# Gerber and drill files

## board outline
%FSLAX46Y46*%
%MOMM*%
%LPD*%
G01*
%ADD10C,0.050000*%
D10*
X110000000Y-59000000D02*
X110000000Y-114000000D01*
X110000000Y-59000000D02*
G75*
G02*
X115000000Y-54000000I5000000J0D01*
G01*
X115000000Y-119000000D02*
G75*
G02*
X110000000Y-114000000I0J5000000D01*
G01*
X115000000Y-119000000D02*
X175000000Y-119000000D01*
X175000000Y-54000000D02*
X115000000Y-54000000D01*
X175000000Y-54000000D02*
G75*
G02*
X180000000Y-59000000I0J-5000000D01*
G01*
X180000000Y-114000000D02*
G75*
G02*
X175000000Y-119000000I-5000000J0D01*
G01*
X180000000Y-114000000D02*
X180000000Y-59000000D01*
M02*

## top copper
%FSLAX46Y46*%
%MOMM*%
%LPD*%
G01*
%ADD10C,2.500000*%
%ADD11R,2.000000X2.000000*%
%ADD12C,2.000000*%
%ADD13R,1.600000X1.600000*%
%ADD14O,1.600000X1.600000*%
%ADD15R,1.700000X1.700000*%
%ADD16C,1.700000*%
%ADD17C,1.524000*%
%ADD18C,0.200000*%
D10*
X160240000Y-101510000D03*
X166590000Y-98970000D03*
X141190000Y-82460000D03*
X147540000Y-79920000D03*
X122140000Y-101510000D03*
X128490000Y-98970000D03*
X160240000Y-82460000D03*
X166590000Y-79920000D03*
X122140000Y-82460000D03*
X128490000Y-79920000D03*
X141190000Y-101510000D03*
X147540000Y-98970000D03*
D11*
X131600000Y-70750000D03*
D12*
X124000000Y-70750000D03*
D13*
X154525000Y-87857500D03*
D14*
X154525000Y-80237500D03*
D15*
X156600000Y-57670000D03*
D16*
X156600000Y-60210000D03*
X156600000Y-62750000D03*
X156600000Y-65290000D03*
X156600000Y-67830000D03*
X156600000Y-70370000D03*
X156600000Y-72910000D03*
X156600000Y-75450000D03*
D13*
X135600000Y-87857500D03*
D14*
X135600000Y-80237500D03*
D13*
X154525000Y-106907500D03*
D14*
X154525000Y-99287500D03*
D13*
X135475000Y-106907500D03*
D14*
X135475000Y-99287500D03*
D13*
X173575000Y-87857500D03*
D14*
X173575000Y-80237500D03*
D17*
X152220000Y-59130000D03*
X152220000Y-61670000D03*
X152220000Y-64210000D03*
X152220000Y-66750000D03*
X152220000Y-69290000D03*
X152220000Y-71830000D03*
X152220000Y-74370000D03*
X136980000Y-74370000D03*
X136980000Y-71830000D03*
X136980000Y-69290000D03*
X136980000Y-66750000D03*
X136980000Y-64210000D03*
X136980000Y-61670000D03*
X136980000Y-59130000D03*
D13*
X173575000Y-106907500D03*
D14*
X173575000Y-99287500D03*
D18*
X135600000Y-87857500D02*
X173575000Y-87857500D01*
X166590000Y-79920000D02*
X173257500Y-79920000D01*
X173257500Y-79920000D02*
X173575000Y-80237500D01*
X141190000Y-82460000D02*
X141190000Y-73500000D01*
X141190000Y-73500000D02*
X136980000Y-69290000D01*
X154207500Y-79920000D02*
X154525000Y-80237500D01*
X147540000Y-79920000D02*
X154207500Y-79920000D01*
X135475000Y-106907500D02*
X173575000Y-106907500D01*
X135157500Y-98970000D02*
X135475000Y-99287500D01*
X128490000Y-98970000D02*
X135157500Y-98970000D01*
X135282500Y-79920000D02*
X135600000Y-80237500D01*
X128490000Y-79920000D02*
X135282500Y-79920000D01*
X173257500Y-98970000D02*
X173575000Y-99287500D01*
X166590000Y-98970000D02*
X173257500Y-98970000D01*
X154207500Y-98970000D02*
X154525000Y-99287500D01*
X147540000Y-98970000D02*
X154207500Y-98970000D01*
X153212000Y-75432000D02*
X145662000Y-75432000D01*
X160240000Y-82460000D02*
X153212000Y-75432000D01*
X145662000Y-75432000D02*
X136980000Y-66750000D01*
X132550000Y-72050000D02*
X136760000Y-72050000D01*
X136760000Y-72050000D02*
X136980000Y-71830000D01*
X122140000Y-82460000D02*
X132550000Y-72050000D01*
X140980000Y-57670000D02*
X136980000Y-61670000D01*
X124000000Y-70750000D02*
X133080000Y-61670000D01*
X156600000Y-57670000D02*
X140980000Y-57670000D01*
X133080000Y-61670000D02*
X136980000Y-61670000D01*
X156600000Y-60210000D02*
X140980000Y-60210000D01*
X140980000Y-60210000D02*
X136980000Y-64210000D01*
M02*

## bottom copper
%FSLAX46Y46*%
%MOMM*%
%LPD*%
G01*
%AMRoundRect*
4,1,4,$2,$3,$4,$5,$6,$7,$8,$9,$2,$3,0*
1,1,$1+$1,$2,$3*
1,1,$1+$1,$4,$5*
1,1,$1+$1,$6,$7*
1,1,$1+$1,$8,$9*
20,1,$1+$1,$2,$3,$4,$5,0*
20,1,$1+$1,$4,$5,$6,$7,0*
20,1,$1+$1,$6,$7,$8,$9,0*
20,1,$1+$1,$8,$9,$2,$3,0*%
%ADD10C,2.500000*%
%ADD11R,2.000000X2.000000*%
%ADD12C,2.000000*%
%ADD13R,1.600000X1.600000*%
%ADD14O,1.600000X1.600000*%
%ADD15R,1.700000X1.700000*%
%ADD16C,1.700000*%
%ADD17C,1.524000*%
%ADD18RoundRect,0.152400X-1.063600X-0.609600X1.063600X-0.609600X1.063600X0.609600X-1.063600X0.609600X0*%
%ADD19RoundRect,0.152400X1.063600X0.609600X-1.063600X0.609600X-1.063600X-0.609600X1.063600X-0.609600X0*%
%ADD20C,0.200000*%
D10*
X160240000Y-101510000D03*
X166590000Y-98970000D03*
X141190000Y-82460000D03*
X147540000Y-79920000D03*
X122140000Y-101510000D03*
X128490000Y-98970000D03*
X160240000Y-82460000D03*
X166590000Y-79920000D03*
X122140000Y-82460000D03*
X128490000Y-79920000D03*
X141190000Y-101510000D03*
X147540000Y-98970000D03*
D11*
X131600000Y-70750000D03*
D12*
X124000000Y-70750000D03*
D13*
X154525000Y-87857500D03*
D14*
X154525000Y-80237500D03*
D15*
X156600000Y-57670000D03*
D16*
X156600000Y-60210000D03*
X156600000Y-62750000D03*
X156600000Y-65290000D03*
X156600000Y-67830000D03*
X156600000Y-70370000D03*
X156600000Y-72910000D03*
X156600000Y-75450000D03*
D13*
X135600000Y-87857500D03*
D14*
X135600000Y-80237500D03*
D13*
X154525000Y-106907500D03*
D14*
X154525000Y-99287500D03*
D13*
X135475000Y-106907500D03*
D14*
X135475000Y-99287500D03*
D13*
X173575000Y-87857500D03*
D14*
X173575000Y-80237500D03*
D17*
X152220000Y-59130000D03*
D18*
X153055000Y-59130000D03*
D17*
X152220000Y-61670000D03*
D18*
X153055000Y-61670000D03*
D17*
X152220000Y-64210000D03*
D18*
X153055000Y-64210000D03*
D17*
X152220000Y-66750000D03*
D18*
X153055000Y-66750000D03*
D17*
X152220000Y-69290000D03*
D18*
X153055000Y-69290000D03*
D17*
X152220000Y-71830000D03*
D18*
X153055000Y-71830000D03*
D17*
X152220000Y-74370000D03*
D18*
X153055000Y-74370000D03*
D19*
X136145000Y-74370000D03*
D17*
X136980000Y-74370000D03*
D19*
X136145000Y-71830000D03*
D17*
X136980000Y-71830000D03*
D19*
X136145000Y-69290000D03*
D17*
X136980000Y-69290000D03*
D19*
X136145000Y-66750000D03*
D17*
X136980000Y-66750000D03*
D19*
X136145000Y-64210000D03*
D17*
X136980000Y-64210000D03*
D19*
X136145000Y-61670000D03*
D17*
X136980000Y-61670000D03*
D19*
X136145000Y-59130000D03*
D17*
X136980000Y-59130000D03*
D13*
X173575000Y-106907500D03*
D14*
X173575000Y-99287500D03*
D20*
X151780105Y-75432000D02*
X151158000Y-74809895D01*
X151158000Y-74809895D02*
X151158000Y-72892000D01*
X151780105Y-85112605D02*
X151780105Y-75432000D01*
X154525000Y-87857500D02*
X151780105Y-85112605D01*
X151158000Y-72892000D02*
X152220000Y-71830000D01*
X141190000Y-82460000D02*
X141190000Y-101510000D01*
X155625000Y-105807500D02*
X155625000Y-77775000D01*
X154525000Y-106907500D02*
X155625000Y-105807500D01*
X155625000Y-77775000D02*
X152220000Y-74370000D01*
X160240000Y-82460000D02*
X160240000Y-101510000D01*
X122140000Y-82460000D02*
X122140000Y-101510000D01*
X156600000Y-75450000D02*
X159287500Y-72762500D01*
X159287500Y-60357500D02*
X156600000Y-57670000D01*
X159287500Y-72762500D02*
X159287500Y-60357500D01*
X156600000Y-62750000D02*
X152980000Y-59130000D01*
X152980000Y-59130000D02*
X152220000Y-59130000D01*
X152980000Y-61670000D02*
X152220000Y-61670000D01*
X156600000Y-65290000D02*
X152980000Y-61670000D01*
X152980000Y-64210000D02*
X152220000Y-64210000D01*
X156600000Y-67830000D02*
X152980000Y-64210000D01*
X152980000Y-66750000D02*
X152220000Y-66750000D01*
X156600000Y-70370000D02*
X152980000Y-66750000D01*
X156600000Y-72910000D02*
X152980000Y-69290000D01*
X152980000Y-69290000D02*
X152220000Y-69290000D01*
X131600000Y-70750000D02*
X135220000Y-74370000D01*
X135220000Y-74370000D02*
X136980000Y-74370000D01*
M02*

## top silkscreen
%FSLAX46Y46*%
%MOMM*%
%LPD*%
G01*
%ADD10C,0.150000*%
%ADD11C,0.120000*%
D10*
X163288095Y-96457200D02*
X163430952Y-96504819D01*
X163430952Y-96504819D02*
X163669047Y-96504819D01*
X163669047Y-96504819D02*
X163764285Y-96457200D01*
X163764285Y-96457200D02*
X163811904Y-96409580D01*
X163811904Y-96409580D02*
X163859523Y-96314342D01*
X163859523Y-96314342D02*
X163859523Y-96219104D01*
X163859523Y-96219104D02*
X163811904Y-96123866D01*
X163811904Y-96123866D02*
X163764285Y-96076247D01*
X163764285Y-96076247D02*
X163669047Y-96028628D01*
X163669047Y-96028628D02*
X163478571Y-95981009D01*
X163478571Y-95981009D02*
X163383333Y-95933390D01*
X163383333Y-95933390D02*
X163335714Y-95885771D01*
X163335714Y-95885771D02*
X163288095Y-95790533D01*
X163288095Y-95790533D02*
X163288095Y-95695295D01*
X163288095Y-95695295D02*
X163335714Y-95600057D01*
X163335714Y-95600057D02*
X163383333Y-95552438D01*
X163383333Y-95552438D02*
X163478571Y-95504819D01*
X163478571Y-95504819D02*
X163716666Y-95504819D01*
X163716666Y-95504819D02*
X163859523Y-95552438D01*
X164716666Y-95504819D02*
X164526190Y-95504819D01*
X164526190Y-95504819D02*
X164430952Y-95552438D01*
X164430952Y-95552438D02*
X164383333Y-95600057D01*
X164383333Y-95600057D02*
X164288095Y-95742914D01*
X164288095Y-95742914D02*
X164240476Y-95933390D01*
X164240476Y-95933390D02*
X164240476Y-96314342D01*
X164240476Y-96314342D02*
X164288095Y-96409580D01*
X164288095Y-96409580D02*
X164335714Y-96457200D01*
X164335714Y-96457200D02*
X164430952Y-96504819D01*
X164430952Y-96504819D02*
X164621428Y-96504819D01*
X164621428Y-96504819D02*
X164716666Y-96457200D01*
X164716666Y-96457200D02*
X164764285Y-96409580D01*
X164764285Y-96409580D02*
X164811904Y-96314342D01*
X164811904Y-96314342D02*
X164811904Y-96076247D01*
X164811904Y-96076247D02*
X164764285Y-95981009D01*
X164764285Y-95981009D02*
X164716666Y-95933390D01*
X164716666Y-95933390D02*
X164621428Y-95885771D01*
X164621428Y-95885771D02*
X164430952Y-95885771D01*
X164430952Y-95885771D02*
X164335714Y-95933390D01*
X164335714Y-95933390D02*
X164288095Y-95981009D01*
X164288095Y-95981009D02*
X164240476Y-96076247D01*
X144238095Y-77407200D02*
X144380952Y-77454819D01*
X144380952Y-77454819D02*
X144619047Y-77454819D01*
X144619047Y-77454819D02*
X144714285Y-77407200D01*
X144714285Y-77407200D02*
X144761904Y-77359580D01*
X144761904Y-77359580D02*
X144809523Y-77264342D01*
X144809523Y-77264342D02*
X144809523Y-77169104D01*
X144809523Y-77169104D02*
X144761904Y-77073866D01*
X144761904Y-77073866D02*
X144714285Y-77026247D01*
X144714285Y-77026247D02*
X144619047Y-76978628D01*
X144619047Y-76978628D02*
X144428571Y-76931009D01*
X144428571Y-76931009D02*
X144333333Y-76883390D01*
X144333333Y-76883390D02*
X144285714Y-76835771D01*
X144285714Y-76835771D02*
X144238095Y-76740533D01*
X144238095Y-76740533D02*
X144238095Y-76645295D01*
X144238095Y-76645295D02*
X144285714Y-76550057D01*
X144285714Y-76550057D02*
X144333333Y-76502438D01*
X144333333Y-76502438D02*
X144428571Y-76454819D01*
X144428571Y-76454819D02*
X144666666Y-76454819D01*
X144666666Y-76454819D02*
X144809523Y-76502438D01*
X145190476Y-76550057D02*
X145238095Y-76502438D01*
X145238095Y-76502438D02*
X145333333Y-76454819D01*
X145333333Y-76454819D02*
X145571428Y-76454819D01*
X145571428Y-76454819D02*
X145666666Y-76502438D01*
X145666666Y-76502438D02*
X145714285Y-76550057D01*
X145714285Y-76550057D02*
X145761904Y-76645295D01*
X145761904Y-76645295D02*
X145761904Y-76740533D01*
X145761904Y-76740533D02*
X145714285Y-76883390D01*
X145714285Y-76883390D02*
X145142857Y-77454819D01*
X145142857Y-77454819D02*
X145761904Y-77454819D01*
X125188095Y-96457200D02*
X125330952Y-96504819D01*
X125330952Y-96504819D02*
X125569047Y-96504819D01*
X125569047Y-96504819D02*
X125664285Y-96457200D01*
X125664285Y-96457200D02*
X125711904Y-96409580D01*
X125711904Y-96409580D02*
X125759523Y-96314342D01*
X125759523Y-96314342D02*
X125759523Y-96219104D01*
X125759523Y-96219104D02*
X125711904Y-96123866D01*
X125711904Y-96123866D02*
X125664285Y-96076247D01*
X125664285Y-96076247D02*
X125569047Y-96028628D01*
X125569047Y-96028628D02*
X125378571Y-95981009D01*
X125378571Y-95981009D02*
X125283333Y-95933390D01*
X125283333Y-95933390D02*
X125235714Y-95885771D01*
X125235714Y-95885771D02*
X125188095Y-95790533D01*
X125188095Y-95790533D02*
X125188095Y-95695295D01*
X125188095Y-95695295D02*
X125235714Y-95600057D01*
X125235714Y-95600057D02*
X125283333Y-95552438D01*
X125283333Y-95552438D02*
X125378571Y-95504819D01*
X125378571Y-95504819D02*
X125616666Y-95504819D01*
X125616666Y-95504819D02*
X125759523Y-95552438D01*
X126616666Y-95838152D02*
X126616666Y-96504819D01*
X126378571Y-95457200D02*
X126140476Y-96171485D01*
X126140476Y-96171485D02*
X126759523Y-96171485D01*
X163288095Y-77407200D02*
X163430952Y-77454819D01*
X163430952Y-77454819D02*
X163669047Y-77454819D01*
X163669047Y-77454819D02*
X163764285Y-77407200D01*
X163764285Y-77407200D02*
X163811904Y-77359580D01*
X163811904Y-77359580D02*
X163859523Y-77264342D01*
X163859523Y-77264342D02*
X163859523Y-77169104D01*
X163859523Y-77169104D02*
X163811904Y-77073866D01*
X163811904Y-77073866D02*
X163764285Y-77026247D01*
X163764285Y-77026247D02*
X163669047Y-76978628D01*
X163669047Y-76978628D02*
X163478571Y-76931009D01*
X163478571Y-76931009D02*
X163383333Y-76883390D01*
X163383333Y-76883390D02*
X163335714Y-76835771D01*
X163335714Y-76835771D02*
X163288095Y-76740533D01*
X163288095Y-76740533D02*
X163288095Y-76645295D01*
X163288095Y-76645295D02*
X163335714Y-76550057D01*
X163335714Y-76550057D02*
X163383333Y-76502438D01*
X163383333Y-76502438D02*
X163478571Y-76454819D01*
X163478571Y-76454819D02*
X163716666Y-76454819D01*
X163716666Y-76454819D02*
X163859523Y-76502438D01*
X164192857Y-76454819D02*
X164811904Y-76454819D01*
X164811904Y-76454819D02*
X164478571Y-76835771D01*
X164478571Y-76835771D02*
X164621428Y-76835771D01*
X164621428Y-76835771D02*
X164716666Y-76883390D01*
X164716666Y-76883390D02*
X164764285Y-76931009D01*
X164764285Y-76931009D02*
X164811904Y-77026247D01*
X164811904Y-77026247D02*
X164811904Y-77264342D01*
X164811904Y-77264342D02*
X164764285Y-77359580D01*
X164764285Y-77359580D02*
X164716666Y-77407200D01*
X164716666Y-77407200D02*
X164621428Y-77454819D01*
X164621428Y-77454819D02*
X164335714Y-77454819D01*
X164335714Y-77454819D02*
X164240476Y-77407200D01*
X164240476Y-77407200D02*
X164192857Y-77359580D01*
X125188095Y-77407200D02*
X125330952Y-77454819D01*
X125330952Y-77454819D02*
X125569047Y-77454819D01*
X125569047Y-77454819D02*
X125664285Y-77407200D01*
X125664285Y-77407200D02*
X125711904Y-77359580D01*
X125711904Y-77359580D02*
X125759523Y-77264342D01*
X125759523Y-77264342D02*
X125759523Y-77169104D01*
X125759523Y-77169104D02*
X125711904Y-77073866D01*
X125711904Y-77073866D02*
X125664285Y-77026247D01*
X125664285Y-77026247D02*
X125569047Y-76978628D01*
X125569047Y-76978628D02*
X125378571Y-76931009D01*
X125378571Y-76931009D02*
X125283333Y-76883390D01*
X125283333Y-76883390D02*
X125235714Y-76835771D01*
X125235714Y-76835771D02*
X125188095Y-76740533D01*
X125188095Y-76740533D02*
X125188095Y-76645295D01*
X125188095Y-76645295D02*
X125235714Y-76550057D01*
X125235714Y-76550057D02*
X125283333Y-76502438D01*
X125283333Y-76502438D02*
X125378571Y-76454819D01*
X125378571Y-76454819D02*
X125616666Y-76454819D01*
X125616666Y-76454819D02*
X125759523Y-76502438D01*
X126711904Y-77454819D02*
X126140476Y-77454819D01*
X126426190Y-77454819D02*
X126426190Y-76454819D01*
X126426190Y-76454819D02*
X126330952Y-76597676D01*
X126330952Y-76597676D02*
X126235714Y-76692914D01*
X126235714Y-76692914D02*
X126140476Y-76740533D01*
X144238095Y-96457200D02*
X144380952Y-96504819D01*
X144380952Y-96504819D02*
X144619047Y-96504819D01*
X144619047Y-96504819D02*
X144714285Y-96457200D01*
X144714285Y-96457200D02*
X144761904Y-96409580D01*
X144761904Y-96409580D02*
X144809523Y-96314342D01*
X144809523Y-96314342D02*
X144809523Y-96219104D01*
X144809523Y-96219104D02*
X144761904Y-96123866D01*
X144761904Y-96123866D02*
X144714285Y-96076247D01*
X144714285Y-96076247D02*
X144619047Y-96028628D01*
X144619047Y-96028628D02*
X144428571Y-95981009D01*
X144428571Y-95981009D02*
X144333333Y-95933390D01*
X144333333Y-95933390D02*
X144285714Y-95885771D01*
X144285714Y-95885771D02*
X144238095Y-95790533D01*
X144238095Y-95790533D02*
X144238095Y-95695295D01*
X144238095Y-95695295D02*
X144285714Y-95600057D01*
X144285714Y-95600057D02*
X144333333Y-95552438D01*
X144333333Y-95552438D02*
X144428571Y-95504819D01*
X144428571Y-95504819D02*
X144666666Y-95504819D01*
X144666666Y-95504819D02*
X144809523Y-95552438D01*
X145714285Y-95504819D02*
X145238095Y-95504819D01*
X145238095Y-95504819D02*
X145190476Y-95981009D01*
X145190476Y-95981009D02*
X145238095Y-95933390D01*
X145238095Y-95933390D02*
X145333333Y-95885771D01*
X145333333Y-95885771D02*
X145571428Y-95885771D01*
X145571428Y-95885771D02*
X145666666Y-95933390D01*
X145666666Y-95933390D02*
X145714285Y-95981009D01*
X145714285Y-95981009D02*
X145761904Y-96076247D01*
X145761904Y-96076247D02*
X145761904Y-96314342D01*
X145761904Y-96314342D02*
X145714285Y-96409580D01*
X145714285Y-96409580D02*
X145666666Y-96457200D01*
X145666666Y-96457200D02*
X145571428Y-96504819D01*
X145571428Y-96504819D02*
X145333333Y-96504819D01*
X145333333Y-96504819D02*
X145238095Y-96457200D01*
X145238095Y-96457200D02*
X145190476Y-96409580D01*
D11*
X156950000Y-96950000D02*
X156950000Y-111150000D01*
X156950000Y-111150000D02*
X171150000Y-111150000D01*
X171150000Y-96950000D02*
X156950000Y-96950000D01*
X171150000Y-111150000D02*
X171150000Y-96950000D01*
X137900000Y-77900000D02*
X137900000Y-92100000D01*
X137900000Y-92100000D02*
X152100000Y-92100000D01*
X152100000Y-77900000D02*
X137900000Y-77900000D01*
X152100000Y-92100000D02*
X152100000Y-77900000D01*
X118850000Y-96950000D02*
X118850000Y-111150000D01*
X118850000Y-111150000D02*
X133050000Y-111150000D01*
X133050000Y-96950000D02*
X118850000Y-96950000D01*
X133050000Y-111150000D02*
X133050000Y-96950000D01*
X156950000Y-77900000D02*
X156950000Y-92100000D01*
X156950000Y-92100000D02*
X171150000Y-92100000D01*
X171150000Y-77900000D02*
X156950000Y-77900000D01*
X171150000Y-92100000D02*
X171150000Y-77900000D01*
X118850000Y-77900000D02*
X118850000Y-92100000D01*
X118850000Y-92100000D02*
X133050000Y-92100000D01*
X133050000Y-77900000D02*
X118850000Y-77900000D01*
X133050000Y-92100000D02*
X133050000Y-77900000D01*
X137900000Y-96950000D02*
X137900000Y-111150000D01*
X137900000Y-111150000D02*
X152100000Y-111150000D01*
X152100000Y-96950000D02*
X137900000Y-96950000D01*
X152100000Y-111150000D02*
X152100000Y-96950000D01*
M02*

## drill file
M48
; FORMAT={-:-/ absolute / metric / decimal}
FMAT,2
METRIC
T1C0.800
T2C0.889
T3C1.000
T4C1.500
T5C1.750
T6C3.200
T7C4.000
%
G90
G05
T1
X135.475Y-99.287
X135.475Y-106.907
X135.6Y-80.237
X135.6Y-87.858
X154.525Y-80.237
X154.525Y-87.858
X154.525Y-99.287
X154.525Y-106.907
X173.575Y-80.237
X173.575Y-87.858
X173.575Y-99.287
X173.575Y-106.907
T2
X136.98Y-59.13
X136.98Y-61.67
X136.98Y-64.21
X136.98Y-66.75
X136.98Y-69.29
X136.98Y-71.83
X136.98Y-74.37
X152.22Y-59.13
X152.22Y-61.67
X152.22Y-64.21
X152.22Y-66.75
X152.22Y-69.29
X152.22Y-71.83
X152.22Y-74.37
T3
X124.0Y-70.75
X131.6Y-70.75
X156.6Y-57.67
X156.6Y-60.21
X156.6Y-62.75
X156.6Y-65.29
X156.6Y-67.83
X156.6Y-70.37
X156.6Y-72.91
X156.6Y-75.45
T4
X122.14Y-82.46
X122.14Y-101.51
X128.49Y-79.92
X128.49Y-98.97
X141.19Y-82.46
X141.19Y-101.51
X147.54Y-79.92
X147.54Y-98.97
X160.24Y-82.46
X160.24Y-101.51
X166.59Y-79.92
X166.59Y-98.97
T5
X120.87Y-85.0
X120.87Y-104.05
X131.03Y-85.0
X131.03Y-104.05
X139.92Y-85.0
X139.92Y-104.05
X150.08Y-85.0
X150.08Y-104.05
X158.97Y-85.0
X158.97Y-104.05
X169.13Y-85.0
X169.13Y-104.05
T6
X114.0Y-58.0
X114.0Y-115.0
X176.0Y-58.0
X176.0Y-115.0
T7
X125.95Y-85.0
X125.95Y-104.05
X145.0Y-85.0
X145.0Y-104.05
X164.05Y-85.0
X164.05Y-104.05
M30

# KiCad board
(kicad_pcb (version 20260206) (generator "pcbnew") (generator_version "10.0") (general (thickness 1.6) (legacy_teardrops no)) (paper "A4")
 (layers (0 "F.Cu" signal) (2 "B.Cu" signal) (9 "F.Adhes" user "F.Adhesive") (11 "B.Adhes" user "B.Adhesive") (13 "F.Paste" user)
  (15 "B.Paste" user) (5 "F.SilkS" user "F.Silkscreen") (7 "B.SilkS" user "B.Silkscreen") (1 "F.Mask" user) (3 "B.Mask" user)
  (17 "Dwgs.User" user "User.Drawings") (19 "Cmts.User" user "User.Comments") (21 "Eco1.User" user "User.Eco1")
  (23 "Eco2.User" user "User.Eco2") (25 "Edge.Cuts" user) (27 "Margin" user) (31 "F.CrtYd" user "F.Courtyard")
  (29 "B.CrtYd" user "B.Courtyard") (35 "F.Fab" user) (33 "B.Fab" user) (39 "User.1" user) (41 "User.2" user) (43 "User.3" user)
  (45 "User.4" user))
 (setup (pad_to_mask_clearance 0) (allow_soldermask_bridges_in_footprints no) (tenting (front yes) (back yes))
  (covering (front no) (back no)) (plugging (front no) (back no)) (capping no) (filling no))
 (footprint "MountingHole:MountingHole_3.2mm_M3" (layer "F.Cu") (at 176 58)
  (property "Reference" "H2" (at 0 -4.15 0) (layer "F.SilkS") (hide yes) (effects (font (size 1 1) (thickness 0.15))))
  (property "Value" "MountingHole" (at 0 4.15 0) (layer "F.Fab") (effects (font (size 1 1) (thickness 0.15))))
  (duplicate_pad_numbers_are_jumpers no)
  (pad "" np_thru_hole circle (at 0 0) (size 3.2 3.2) (drill 3.2) (layers "*.Cu" "*.Mask")))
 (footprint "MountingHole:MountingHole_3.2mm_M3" (layer "F.Cu") (at 114 58)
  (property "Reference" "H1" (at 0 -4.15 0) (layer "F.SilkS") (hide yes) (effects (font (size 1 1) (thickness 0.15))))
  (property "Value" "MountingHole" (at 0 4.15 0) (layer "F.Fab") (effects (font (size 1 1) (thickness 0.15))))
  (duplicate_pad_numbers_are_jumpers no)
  (pad "" np_thru_hole circle (at 0 0) (size 3.2 3.2) (drill 3.2) (layers "*.Cu" "*.Mask")))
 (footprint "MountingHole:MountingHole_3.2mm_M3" (layer "F.Cu") (at 176 115)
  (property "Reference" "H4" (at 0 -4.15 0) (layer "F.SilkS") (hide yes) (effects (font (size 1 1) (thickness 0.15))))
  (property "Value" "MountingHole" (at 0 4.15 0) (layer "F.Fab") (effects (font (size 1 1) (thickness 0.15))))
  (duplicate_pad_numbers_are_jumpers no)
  (pad "" np_thru_hole circle (at 0 0) (size 3.2 3.2) (drill 3.2) (layers "*.Cu" "*.Mask")))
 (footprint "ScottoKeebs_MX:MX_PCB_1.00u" (layer "F.Cu") (at 164.05 104.05)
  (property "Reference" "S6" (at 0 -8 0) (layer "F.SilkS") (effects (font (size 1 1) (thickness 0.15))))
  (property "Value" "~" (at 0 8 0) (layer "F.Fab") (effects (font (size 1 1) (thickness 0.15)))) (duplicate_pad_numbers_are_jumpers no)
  (fp_line (start -7.1 -7.1) (end -7.1 7.1) (stroke (width 0.12) (type solid)) (layer "F.SilkS"))
  (fp_line (start -7.1 7.1) (end 7.1 7.1) (stroke (width 0.12) (type solid)) (layer "F.SilkS"))
  (fp_line (start 7.1 -7.1) (end -7.1 -7.1) (stroke (width 0.12) (type solid)) (layer "F.SilkS"))
  (fp_line (start 7.1 7.1) (end 7.1 -7.1) (stroke (width 0.12) (type solid)) (layer "F.SilkS"))
  (pad "" np_thru_hole circle (at -5.08 0) (size 1.75 1.75) (drill 1.75) (layers "*.Cu" "*.Mask"))
  (pad "" np_thru_hole circle (at 0 0) (size 4 4) (drill 4) (layers "*.Cu" "*.Mask"))
  (pad "" np_thru_hole circle (at 5.08 0) (size 1.75 1.75) (drill 1.75) (layers "*.Cu" "*.Mask"))
  (pad "1" thru_hole circle (at -3.81 -2.54) (size 2.5 2.5) (drill 1.5) (layers "*.Cu" "*.Mask") (remove_unused_layers no) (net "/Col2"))
  (pad "2" thru_hole circle (at 2.54 -5.08) (size 2.5 2.5) (drill 1.5) (layers "*.Cu" "*.Mask") (remove_unused_layers no) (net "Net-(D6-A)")))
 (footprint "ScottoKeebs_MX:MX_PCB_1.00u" (layer "F.Cu") (at 145 85)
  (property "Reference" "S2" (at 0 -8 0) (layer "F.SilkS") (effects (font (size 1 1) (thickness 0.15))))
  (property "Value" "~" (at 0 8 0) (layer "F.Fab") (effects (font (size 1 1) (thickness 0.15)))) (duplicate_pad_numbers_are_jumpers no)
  (fp_line (start -7.1 -7.1) (end -7.1 7.1) (stroke (width 0.12) (type solid)) (layer "F.SilkS"))
  (fp_line (start -7.1 7.1) (end 7.1 7.1) (stroke (width 0.12) (type solid)) (layer "F.SilkS"))
  (fp_line (start 7.1 -7.1) (end -7.1 -7.1) (stroke (width 0.12) (type solid)) (layer "F.SilkS"))
  (fp_line (start 7.1 7.1) (end 7.1 -7.1) (stroke (width 0.12) (type solid)) (layer "F.SilkS"))
  (pad "" np_thru_hole circle (at -5.08 0) (size 1.75 1.75) (drill 1.75) (layers "*.Cu" "*.Mask"))
  (pad "" np_thru_hole circle (at 0 0) (size 4 4) (drill 4) (layers "*.Cu" "*.Mask"))
  (pad "" np_thru_hole circle (at 5.08 0) (size 1.75 1.75) (drill 1.75) (layers "*.Cu" "*.Mask"))
  (pad "1" thru_hole circle (at -3.81 -2.54) (size 2.5 2.5) (drill 1.5) (layers "*.Cu" "*.Mask") (remove_unused_layers no) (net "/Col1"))
  (pad "2" thru_hole circle (at 2.54 -5.08) (size 2.5 2.5) (drill 1.5) (layers "*.Cu" "*.Mask") (remove_unused_layers no) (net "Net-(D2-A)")))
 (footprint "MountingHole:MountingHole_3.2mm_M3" (layer "F.Cu") (at 114 115)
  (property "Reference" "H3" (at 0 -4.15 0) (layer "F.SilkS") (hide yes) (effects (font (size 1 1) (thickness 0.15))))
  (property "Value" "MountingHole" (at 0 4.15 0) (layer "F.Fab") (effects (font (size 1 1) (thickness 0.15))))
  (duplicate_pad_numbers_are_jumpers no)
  (pad "" np_thru_hole circle (at 0 0) (size 3.2 3.2) (drill 3.2) (layers "*.Cu" "*.Mask")))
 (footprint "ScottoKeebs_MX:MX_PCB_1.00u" (layer "F.Cu") (at 125.95 104.05)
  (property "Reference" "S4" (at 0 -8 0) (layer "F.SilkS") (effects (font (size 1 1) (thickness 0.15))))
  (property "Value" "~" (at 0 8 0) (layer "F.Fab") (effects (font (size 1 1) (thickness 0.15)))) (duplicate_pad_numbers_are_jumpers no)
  (fp_line (start -7.1 -7.1) (end -7.1 7.1) (stroke (width 0.12) (type solid)) (layer "F.SilkS"))
  (fp_line (start -7.1 7.1) (end 7.1 7.1) (stroke (width 0.12) (type solid)) (layer "F.SilkS"))
  (fp_line (start 7.1 -7.1) (end -7.1 -7.1) (stroke (width 0.12) (type solid)) (layer "F.SilkS"))
  (fp_line (start 7.1 7.1) (end 7.1 -7.1) (stroke (width 0.12) (type solid)) (layer "F.SilkS"))
  (pad "" np_thru_hole circle (at -5.08 0) (size 1.75 1.75) (drill 1.75) (layers "*.Cu" "*.Mask"))
  (pad "" np_thru_hole circle (at 0 0) (size 4 4) (drill 4) (layers "*.Cu" "*.Mask"))
  (pad "" np_thru_hole circle (at 5.08 0) (size 1.75 1.75) (drill 1.75) (layers "*.Cu" "*.Mask"))
  (pad "1" thru_hole circle (at -3.81 -2.54) (size 2.5 2.5) (drill 1.5) (layers "*.Cu" "*.Mask") (remove_unused_layers no) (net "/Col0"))
  (pad "2" thru_hole circle (at 2.54 -5.08) (size 2.5 2.5) (drill 1.5) (layers "*.Cu" "*.Mask") (remove_unused_layers no) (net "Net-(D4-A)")))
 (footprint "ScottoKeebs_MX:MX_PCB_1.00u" (layer "F.Cu") (at 164.05 85)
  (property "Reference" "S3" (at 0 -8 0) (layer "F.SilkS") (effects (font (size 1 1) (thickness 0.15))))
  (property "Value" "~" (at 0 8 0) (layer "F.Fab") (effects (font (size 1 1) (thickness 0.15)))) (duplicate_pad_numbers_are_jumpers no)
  (fp_line (start -7.1 -7.1) (end -7.1 7.1) (stroke (width 0.12) (type solid)) (layer "F.SilkS"))
  (fp_line (start -7.1 7.1) (end 7.1 7.1) (stroke (width 0.12) (type solid)) (layer "F.SilkS"))
  (fp_line (start 7.1 -7.1) (end -7.1 -7.1) (stroke (width 0.12) (type solid)) (layer "F.SilkS"))
  (fp_line (start 7.1 7.1) (end 7.1 -7.1) (stroke (width 0.12) (type solid)) (layer "F.SilkS"))
  (pad "" np_thru_hole circle (at -5.08 0) (size 1.75 1.75) (drill 1.75) (layers "*.Cu" "*.Mask"))
  (pad "" np_thru_hole circle (at 0 0) (size 4 4) (drill 4) (layers "*.Cu" "*.Mask"))
  (pad "" np_thru_hole circle (at 5.08 0) (size 1.75 1.75) (drill 1.75) (layers "*.Cu" "*.Mask"))
  (pad "1" thru_hole circle (at -3.81 -2.54) (size 2.5 2.5) (drill 1.5) (layers "*.Cu" "*.Mask") (remove_unused_layers no) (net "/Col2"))
  (pad "2" thru_hole circle (at 2.54 -5.08) (size 2.5 2.5) (drill 1.5) (layers "*.Cu" "*.Mask") (remove_unused_layers no) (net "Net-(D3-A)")))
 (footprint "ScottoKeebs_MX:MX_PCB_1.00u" (layer "F.Cu") (at 125.95 85)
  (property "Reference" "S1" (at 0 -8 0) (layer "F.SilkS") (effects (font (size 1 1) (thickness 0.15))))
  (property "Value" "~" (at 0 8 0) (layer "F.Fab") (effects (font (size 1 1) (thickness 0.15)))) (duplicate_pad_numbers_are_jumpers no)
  (fp_line (start -7.1 -7.1) (end -7.1 7.1) (stroke (width 0.12) (type solid)) (layer "F.SilkS"))
  (fp_line (start -7.1 7.1) (end 7.1 7.1) (stroke (width 0.12) (type solid)) (layer "F.SilkS"))
  (fp_line (start 7.1 -7.1) (end -7.1 -7.1) (stroke (width 0.12) (type solid)) (layer "F.SilkS"))
  (fp_line (start 7.1 7.1) (end 7.1 -7.1) (stroke (width 0.12) (type solid)) (layer "F.SilkS"))
  (pad "" np_thru_hole circle (at -5.08 0) (size 1.75 1.75) (drill 1.75) (layers "*.Cu" "*.Mask"))
  (pad "" np_thru_hole circle (at 0 0) (size 4 4) (drill 4) (layers "*.Cu" "*.Mask"))
  (pad "" np_thru_hole circle (at 5.08 0) (size 1.75 1.75) (drill 1.75) (layers "*.Cu" "*.Mask"))
  (pad "1" thru_hole circle (at -3.81 -2.54) (size 2.5 2.5) (drill 1.5) (layers "*.Cu" "*.Mask") (remove_unused_layers no) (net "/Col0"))
  (pad "2" thru_hole circle (at 2.54 -5.08) (size 2.5 2.5) (drill 1.5) (layers "*.Cu" "*.Mask") (remove_unused_layers no) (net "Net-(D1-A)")))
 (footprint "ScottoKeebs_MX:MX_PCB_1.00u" (layer "F.Cu") (at 145 104.05)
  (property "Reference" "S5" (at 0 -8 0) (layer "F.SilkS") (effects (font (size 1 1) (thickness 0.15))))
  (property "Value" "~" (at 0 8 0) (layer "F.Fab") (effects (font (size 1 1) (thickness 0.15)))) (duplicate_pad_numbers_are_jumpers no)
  (fp_line (start -7.1 -7.1) (end -7.1 7.1) (stroke (width 0.12) (type solid)) (layer "F.SilkS"))
  (fp_line (start -7.1 7.1) (end 7.1 7.1) (stroke (width 0.12) (type solid)) (layer "F.SilkS"))
  (fp_line (start 7.1 -7.1) (end -7.1 -7.1) (stroke (width 0.12) (type solid)) (layer "F.SilkS"))
  (fp_line (start 7.1 7.1) (end 7.1 -7.1) (stroke (width 0.12) (type solid)) (layer "F.SilkS"))
  (pad "" np_thru_hole circle (at -5.08 0) (size 1.75 1.75) (drill 1.75) (layers "*.Cu" "*.Mask"))
  (pad "" np_thru_hole circle (at 0 0) (size 4 4) (drill 4) (layers "*.Cu" "*.Mask"))
  (pad "" np_thru_hole circle (at 5.08 0) (size 1.75 1.75) (drill 1.75) (layers "*.Cu" "*.Mask"))
  (pad "1" thru_hole circle (at -3.81 -2.54) (size 2.5 2.5) (drill 1.5) (layers "*.Cu" "*.Mask") (remove_unused_layers no) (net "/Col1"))
  (pad "2" thru_hole circle (at 2.54 -5.08) (size 2.5 2.5) (drill 1.5) (layers "*.Cu" "*.Mask") (remove_unused_layers no) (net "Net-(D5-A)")))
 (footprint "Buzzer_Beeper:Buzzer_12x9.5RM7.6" (layer "B.Cu") (at 131.6 70.75 180)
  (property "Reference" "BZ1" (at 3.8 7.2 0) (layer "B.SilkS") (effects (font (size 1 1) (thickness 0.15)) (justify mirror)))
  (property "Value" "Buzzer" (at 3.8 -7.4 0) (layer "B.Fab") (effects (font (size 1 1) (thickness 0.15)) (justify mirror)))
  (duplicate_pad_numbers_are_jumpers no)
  (pad "1" thru_hole rect (at 0 0 180) (size 2 2) (drill 1) (layers "*.Cu" "*.Mask") (remove_unused_layers no) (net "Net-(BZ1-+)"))
  (pad "2" thru_hole circle (at 7.6 0 180) (size 2 2) (drill 1) (layers "*.Cu" "*.Mask") (remove_unused_layers no) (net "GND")))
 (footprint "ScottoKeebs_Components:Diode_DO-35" (layer "B.Cu") (at 154.525 87.8575 90)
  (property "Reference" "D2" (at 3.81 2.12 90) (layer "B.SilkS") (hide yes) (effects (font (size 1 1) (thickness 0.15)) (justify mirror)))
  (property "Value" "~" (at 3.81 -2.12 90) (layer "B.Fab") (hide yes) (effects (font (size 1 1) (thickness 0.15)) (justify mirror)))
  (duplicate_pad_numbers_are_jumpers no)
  (pad "1" thru_hole rect (at 0 0 90) (size 1.6 1.6) (drill 0.8) (layers "*.Cu" "*.Mask") (remove_unused_layers no) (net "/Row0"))
  (pad "2" thru_hole oval (at 7.62 0 90) (size 1.6 1.6) (drill 0.8) (layers "*.Cu" "*.Mask") (remove_unused_layers no) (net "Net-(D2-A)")))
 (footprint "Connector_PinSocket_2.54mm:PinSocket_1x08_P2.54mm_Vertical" (layer "B.Cu") (at 156.6 57.67 180)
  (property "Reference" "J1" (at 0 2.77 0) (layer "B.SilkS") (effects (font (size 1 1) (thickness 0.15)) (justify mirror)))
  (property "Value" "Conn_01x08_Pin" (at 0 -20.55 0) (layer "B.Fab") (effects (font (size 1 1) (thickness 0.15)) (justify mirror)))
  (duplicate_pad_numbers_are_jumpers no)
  (pad "1" thru_hole rect (at 0 0 180) (size 1.7 1.7) (drill 1) (layers "*.Cu" "*.Mask") (remove_unused_layers no) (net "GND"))
  (pad "2" thru_hole circle (at 0 -2.54 180) (size 1.7 1.7) (drill 1) (layers "*.Cu" "*.Mask") (remove_unused_layers no) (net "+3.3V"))
  (pad "3" thru_hole circle (at 0 -5.08 180) (size 1.7 1.7) (drill 1) (layers "*.Cu" "*.Mask") (remove_unused_layers no) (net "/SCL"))
  (pad "4" thru_hole circle (at 0 -7.62 180) (size 1.7 1.7) (drill 1) (layers "*.Cu" "*.Mask") (remove_unused_layers no) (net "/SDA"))
  (pad "5" thru_hole circle (at 0 -10.16 180) (size 1.7 1.7) (drill 1) (layers "*.Cu" "*.Mask") (remove_unused_layers no) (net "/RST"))
  (pad "6" thru_hole circle (at 0 -12.7 180) (size 1.7 1.7) (drill 1) (layers "*.Cu" "*.Mask") (remove_unused_layers no) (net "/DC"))
  (pad "7" thru_hole circle (at 0 -15.24 180) (size 1.7 1.7) (drill 1) (layers "*.Cu" "*.Mask") (remove_unused_layers no) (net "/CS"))
  (pad "8" thru_hole circle (at 0 -17.78 180) (size 1.7 1.7) (drill 1) (layers "*.Cu" "*.Mask") (remove_unused_layers no) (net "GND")))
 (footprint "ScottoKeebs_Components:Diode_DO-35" (layer "B.Cu") (at 135.6 87.8575 90)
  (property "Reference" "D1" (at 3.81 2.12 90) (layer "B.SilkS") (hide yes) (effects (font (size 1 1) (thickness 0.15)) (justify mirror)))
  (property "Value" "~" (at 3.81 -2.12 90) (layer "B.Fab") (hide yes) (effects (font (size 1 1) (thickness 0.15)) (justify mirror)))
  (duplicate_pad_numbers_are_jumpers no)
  (pad "1" thru_hole rect (at 0 0 90) (size 1.6 1.6) (drill 0.8) (layers "*.Cu" "*.Mask") (remove_unused_layers no) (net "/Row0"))
  (pad "2" thru_hole oval (at 7.62 0 90) (size 1.6 1.6) (drill 0.8) (layers "*.Cu" "*.Mask") (remove_unused_layers no) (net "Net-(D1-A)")))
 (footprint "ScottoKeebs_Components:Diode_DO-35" (layer "B.Cu") (at 154.525 106.9075 90)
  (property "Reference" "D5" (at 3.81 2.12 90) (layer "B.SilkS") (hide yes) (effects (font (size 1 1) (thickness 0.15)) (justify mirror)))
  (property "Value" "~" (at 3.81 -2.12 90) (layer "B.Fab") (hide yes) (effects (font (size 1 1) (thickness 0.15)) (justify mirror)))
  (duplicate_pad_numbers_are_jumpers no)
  (pad "1" thru_hole rect (at 0 0 90) (size 1.6 1.6) (drill 0.8) (layers "*.Cu" "*.Mask") (remove_unused_layers no) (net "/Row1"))
  (pad "2" thru_hole oval (at 7.62 0 90) (size 1.6 1.6) (drill 0.8) (layers "*.Cu" "*.Mask") (remove_unused_layers no) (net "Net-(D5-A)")))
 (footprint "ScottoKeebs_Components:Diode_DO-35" (layer "B.Cu") (at 135.475 106.9075 90)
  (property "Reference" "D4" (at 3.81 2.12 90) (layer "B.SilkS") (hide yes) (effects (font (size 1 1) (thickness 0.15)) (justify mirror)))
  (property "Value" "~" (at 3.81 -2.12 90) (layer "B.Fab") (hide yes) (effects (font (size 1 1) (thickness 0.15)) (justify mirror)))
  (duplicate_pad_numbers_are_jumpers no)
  (pad "1" thru_hole rect (at 0 0 90) (size 1.6 1.6) (drill 0.8) (layers "*.Cu" "*.Mask") (remove_unused_layers no) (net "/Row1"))
  (pad "2" thru_hole oval (at 7.62 0 90) (size 1.6 1.6) (drill 0.8) (layers "*.Cu" "*.Mask") (remove_unused_layers no) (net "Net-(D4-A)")))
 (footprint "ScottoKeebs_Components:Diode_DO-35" (layer "B.Cu") (at 173.575 87.8575 90)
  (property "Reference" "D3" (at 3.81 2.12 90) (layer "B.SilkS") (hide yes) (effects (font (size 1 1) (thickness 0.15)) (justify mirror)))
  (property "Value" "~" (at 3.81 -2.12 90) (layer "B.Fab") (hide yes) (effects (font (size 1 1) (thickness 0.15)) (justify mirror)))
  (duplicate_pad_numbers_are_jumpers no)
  (pad "1" thru_hole rect (at 0 0 90) (size 1.6 1.6) (drill 0.8) (layers "*.Cu" "*.Mask") (remove_unused_layers no) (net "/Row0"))
  (pad "2" thru_hole oval (at 7.62 0 90) (size 1.6 1.6) (drill 0.8) (layers "*.Cu" "*.Mask") (remove_unused_layers no) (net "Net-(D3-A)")))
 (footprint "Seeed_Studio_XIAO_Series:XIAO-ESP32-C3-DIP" (layer "B.Cu") (at 144.6 66.75 90)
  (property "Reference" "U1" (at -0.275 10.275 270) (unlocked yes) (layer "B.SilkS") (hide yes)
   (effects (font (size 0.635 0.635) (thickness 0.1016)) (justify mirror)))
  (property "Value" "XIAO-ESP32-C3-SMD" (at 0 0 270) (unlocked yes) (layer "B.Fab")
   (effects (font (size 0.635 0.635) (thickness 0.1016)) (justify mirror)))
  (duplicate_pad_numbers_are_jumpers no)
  (pad "1" thru_hole circle (at 7.62 7.62) (size 1.524 1.524) (drill 0.889) (layers "*.Cu" "*.Mask") (remove_unused_layers no) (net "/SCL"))
  (pad "1" smd roundrect (at 7.62 8.455) (size 2.432 1.524) (layers "B.Cu" "B.Mask") (roundrect_rratio 0.1) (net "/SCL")
   (thermal_bridge_angle 45))
  (pad "2" thru_hole circle (at 5.08 7.62) (size 1.524 1.524) (drill 0.889) (layers "*.Cu" "*.Mask") (remove_unused_layers no) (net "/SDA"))
  (pad "2" smd roundrect (at 5.08 8.455) (size 2.432 1.524) (layers "B.Cu" "B.Mask") (roundrect_rratio 0.1) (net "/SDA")
   (thermal_bridge_angle 45))
  (pad "3" thru_hole circle (at 2.54 7.62) (size 1.524 1.524) (drill 0.889) (layers "*.Cu" "*.Mask") (remove_unused_layers no) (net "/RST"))
  (pad "3" smd roundrect (at 2.54 8.455) (size 2.432 1.524) (layers "B.Cu" "B.Mask") (roundrect_rratio 0.1) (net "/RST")
   (thermal_bridge_angle 45))
  (pad "4" thru_hole circle (at 0 7.62) (size 1.524 1.524) (drill 0.889) (layers "*.Cu" "*.Mask") (remove_unused_layers no) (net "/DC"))
  (pad "4" smd roundrect (at 0 8.455) (size 2.432 1.524) (layers "B.Cu" "B.Mask") (roundrect_rratio 0.1) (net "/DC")
   (thermal_bridge_angle 45))
  (pad "5" thru_hole circle (at -2.54 7.62) (size 1.524 1.524) (drill 0.889) (layers "*.Cu" "*.Mask") (remove_unused_layers no) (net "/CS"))
  (pad "5" smd roundrect (at -2.54 8.455) (size 2.432 1.524) (layers "B.Cu" "B.Mask") (roundrect_rratio 0.1) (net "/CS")
   (thermal_bridge_angle 45))
  (pad "6" thru_hole circle (at -5.08 7.62) (size 1.524 1.524) (drill 0.889) (layers "*.Cu" "*.Mask") (remove_unused_layers no)
   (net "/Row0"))
  (pad "6" smd roundrect (at -5.08 8.455) (size 2.432 1.524) (layers "B.Cu" "B.Mask") (roundrect_rratio 0.1) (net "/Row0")
   (thermal_bridge_angle 45))
  (pad "7" thru_hole circle (at -7.62 7.62) (size 1.524 1.524) (drill 0.889) (layers "*.Cu" "*.Mask") (remove_unused_layers no)
   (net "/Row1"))
  (pad "7" smd roundrect (at -7.62 8.455) (size 2.432 1.524) (layers "B.Cu" "B.Mask") (roundrect_rratio 0.1) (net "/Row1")
   (thermal_bridge_angle 45))
  (pad "8" smd roundrect (at -7.62 -8.455 180) (size 2.432 1.524) (layers "B.Cu" "B.Mask") (roundrect_rratio 0.1) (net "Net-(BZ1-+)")
   (thermal_bridge_angle 45))
  (pad "8" thru_hole circle (at -7.62 -7.62 180) (size 1.524 1.524) (drill 0.889) (layers "*.Cu" "*.Mask") (remove_unused_layers no)
   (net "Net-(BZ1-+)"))
  (pad "9" smd roundrect (at -5.08 -8.455 180) (size 2.432 1.524) (layers "B.Cu" "B.Mask") (roundrect_rratio 0.1) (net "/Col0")
   (thermal_bridge_angle 45))
  (pad "9" thru_hole circle (at -5.08 -7.62 180) (size 1.524 1.524) (drill 0.889) (layers "*.Cu" "*.Mask") (remove_unused_layers no)
   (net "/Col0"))
  (pad "10" smd roundrect (at -2.54 -8.455 180) (size 2.432 1.524) (layers "B.Cu" "B.Mask") (roundrect_rratio 0.1) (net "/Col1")
   (thermal_bridge_angle 45))
  (pad "10" thru_hole circle (at -2.54 -7.62 180) (size 1.524 1.524) (drill 0.889) (layers "*.Cu" "*.Mask") (remove_unused_layers no)
   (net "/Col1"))
  (pad "11" smd roundrect (at 0 -8.455 180) (size 2.432 1.524) (layers "B.Cu" "B.Mask") (roundrect_rratio 0.1) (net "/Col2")
   (thermal_bridge_angle 45))
  (pad "11" thru_hole circle (at 0 -7.62 180) (size 1.524 1.524) (drill 0.889) (layers "*.Cu" "*.Mask") (remove_unused_layers no)
   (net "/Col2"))
  (pad "12" smd roundrect (at 2.54 -8.455 180) (size 2.432 1.524) (layers "B.Cu" "B.Mask") (roundrect_rratio 0.1) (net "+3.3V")
   (thermal_bridge_angle 45))
  (pad "12" thru_hole circle (at 2.54 -7.62 180) (size 1.524 1.524) (drill 0.889) (layers "*.Cu" "*.Mask") (remove_unused_layers no)
   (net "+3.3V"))
  (pad "13" smd roundrect (at 5.08 -8.455 180) (size 2.432 1.524) (layers "B.Cu" "B.Mask") (roundrect_rratio 0.1) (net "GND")
   (thermal_bridge_angle 45))
  (pad "13" thru_hole circle (at 5.08 -7.62 180) (size 1.524 1.524) (drill 0.889) (layers "*.Cu" "*.Mask") (remove_unused_layers no)
   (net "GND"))
  (pad "14" smd roundrect (at 7.62 -8.455 180) (size 2.432 1.524) (layers "B.Cu" "B.Mask") (roundrect_rratio 0.1)
   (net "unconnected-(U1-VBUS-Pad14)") (thermal_bridge_angle 45))
  (pad "14" thru_hole circle (at 7.62 -7.62 180) (size 1.524 1.524) (drill 0.889) (layers "*.Cu" "*.Mask") (remove_unused_layers no)
   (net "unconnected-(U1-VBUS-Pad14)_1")))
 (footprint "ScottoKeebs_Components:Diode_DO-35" (layer "B.Cu") (at 173.575 106.9075 90)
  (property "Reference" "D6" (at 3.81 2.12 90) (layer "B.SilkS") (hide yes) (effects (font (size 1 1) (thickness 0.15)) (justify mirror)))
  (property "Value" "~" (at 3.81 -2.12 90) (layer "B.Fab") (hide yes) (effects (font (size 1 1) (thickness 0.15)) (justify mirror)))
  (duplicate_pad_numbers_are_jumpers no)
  (pad "1" thru_hole rect (at 0 0 90) (size 1.6 1.6) (drill 0.8) (layers "*.Cu" "*.Mask") (remove_unused_layers no) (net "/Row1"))
  (pad "2" thru_hole oval (at 7.62 0 90) (size 1.6 1.6) (drill 0.8) (layers "*.Cu" "*.Mask") (remove_unused_layers no) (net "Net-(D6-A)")))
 (gr_line (start 110 59) (end 110 114) (stroke (width 0.05) (type default)) (layer "Edge.Cuts"))
 (gr_arc (start 110 59) (mid 111.464466 55.464466) (end 115 54) (stroke (width 0.05) (type default)) (layer "Edge.Cuts"))
 (gr_arc (start 115 119) (mid 111.464466 117.535534) (end 110 114) (stroke (width 0.05) (type default)) (layer "Edge.Cuts"))
 (gr_line (start 115 119) (end 175 119) (stroke (width 0.05) (type default)) (layer "Edge.Cuts"))
 (gr_line (start 175 54) (end 115 54) (stroke (width 0.05) (type default)) (layer "Edge.Cuts"))
 (gr_arc (start 175 54) (mid 178.535534 55.464466) (end 180 59) (stroke (width 0.05) (type default)) (layer "Edge.Cuts"))
 (gr_arc (start 180 114) (mid 178.535534 117.535534) (end 175 119) (stroke (width 0.05) (type default)) (layer "Edge.Cuts"))
 (gr_line (start 180 114) (end 180 59) (stroke (width 0.05) (type default)) (layer "Edge.Cuts"))
 (segment (start 135.6 87.8575) (end 173.575 87.8575) (width 0.2) (layer "F.Cu") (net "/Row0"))
 (segment (start 151.780105 75.432) (end 151.158 74.809895) (width 0.2) (layer "B.Cu") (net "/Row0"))
 (segment (start 151.158 74.809895) (end 151.158 72.892) (width 0.2) (layer "B.Cu") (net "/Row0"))
 (segment (start 151.780105 85.112605) (end 151.780105 75.432) (width 0.2) (layer "B.Cu") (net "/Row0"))
 (segment (start 154.525 87.8575) (end 151.780105 85.112605) (width 0.2) (layer "B.Cu") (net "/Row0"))
 (segment (start 151.158 72.892) (end 152.22 71.83) (width 0.2) (layer "B.Cu") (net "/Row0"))
 (segment (start 166.59 79.92) (end 173.2575 79.92) (width 0.2) (layer "F.Cu") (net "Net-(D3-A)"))
 (segment (start 173.2575 79.92) (end 173.575 80.2375) (width 0.2) (layer "F.Cu") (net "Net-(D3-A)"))
 (segment (start 141.19 82.46) (end 141.19 73.5) (width 0.2) (layer "F.Cu") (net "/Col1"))
 (segment (start 141.19 73.5) (end 136.98 69.29) (width 0.2) (layer "F.Cu") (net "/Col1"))
 (segment (start 141.19 82.46) (end 141.19 101.51) (width 0.2) (layer "B.Cu") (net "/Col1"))
 (segment (start 154.2075 79.92) (end 154.525 80.2375) (width 0.2) (layer "F.Cu") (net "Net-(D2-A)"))
 (segment (start 147.54 79.92) (end 154.2075 79.92) (width 0.2) (layer "F.Cu") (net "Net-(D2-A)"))
 (segment (start 135.475 106.9075) (end 173.575 106.9075) (width 0.2) (layer "F.Cu") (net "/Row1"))
 (segment (start 155.625 105.8075) (end 155.625 77.775) (width 0.2) (layer "B.Cu") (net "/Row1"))
 (segment (start 154.525 106.9075) (end 155.625 105.8075) (width 0.2) (layer "B.Cu") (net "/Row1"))
 (segment (start 155.625 77.775) (end 152.22 74.37) (width 0.2) (layer "B.Cu") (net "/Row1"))
 (segment (start 135.1575 98.97) (end 135.475 99.2875) (width 0.2) (layer "F.Cu") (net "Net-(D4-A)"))
 (segment (start 128.49 98.97) (end 135.1575 98.97) (width 0.2) (layer "F.Cu") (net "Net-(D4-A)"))
 (segment (start 135.2825 79.92) (end 135.6 80.2375) (width 0.2) (layer "F.Cu") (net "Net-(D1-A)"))
 (segment (start 128.49 79.92) (end 135.2825 79.92) (width 0.2) (layer "F.Cu") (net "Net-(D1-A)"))
 (segment (start 173.2575 98.97) (end 173.575 99.2875) (width 0.2) (layer "F.Cu") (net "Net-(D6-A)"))
 (segment (start 166.59 98.97) (end 173.2575 98.97) (width 0.2) (layer "F.Cu") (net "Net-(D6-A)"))
 (segment (start 154.2075 98.97) (end 154.525 99.2875) (width 0.2) (layer "F.Cu") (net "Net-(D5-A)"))
 (segment (start 147.54 98.97) (end 154.2075 98.97) (width 0.2) (layer "F.Cu") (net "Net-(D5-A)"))
 (segment (start 153.212 75.432) (end 145.662 75.432) (width 0.2) (layer "F.Cu") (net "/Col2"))
 (segment (start 160.24 82.46) (end 153.212 75.432) (width 0.2) (layer "F.Cu") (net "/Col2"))
 (segment (start 145.662 75.432) (end 136.98 66.75) (width 0.2) (layer "F.Cu") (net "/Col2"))
 (segment (start 160.24 82.46) (end 160.24 101.51) (width 0.2) (layer "B.Cu") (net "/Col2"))
 (segment (start 132.55 72.05) (end 136.76 72.05) (width 0.2) (layer "F.Cu") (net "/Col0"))
 (segment (start 136.76 72.05) (end 136.98 71.83) (width 0.2) (layer "F.Cu") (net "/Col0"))
 (segment (start 122.14 82.46) (end 132.55 72.05) (width 0.2) (layer "F.Cu") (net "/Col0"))
 (segment (start 122.14 82.46) (end 122.14 101.51) (width 0.2) (layer "B.Cu") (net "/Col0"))
 (segment (start 140.98 57.67) (end 136.98 61.67) (width 0.2) (layer "F.Cu") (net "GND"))
 (segment (start 124 70.75) (end 133.08 61.67) (width 0.2) (layer "F.Cu") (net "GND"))
 (segment (start 156.6 57.67) (end 140.98 57.67) (width 0.2) (layer "F.Cu") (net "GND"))
 (segment (start 133.08 61.67) (end 136.98 61.67) (width 0.2) (layer "F.Cu") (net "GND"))
 (segment (start 156.6 75.45) (end 159.2875 72.7625) (width 0.2) (layer "B.Cu") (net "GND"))
 (segment (start 159.2875 60.3575) (end 156.6 57.67) (width 0.2) (layer "B.Cu") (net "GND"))
 (segment (start 159.2875 72.7625) (end 159.2875 60.3575) (width 0.2) (layer "B.Cu") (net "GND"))
 (segment (start 156.6 60.21) (end 140.98 60.21) (width 0.2) (layer "F.Cu") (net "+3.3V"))
 (segment (start 140.98 60.21) (end 136.98 64.21) (width 0.2) (layer "F.Cu") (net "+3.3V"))
 (segment (start 156.6 62.75) (end 152.98 59.13) (width 0.2) (layer "B.Cu") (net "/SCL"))
 (segment (start 152.98 59.13) (end 152.22 59.13) (width 0.2) (layer "B.Cu") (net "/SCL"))
 (segment (start 152.98 61.67) (end 152.22 61.67) (width 0.2) (layer "B.Cu") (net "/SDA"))
 (segment (start 156.6 65.29) (end 152.98 61.67) (width 0.2) (layer "B.Cu") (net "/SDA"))
 (segment (start 152.98 64.21) (end 152.22 64.21) (width 0.2) (layer "B.Cu") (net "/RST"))
 (segment (start 156.6 67.83) (end 152.98 64.21) (width 0.2) (layer "B.Cu") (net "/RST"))
 (segment (start 152.98 66.75) (end 152.22 66.75) (width 0.2) (layer "B.Cu") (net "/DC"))
 (segment (start 156.6 70.37) (end 152.98 66.75) (width 0.2) (layer "B.Cu") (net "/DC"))
 (segment (start 156.6 72.91) (end 152.98 69.29) (width 0.2) (layer "B.Cu") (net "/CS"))
 (segment (start 152.98 69.29) (end 152.22 69.29) (width 0.2) (layer "B.Cu") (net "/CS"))
 (segment (start 131.6 70.75) (end 135.22 74.37) (width 0.2) (layer "B.Cu") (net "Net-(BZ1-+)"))
 (segment (start 135.22 74.37) (end 136.98 74.37) (width 0.2) (layer "B.Cu") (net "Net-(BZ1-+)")))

